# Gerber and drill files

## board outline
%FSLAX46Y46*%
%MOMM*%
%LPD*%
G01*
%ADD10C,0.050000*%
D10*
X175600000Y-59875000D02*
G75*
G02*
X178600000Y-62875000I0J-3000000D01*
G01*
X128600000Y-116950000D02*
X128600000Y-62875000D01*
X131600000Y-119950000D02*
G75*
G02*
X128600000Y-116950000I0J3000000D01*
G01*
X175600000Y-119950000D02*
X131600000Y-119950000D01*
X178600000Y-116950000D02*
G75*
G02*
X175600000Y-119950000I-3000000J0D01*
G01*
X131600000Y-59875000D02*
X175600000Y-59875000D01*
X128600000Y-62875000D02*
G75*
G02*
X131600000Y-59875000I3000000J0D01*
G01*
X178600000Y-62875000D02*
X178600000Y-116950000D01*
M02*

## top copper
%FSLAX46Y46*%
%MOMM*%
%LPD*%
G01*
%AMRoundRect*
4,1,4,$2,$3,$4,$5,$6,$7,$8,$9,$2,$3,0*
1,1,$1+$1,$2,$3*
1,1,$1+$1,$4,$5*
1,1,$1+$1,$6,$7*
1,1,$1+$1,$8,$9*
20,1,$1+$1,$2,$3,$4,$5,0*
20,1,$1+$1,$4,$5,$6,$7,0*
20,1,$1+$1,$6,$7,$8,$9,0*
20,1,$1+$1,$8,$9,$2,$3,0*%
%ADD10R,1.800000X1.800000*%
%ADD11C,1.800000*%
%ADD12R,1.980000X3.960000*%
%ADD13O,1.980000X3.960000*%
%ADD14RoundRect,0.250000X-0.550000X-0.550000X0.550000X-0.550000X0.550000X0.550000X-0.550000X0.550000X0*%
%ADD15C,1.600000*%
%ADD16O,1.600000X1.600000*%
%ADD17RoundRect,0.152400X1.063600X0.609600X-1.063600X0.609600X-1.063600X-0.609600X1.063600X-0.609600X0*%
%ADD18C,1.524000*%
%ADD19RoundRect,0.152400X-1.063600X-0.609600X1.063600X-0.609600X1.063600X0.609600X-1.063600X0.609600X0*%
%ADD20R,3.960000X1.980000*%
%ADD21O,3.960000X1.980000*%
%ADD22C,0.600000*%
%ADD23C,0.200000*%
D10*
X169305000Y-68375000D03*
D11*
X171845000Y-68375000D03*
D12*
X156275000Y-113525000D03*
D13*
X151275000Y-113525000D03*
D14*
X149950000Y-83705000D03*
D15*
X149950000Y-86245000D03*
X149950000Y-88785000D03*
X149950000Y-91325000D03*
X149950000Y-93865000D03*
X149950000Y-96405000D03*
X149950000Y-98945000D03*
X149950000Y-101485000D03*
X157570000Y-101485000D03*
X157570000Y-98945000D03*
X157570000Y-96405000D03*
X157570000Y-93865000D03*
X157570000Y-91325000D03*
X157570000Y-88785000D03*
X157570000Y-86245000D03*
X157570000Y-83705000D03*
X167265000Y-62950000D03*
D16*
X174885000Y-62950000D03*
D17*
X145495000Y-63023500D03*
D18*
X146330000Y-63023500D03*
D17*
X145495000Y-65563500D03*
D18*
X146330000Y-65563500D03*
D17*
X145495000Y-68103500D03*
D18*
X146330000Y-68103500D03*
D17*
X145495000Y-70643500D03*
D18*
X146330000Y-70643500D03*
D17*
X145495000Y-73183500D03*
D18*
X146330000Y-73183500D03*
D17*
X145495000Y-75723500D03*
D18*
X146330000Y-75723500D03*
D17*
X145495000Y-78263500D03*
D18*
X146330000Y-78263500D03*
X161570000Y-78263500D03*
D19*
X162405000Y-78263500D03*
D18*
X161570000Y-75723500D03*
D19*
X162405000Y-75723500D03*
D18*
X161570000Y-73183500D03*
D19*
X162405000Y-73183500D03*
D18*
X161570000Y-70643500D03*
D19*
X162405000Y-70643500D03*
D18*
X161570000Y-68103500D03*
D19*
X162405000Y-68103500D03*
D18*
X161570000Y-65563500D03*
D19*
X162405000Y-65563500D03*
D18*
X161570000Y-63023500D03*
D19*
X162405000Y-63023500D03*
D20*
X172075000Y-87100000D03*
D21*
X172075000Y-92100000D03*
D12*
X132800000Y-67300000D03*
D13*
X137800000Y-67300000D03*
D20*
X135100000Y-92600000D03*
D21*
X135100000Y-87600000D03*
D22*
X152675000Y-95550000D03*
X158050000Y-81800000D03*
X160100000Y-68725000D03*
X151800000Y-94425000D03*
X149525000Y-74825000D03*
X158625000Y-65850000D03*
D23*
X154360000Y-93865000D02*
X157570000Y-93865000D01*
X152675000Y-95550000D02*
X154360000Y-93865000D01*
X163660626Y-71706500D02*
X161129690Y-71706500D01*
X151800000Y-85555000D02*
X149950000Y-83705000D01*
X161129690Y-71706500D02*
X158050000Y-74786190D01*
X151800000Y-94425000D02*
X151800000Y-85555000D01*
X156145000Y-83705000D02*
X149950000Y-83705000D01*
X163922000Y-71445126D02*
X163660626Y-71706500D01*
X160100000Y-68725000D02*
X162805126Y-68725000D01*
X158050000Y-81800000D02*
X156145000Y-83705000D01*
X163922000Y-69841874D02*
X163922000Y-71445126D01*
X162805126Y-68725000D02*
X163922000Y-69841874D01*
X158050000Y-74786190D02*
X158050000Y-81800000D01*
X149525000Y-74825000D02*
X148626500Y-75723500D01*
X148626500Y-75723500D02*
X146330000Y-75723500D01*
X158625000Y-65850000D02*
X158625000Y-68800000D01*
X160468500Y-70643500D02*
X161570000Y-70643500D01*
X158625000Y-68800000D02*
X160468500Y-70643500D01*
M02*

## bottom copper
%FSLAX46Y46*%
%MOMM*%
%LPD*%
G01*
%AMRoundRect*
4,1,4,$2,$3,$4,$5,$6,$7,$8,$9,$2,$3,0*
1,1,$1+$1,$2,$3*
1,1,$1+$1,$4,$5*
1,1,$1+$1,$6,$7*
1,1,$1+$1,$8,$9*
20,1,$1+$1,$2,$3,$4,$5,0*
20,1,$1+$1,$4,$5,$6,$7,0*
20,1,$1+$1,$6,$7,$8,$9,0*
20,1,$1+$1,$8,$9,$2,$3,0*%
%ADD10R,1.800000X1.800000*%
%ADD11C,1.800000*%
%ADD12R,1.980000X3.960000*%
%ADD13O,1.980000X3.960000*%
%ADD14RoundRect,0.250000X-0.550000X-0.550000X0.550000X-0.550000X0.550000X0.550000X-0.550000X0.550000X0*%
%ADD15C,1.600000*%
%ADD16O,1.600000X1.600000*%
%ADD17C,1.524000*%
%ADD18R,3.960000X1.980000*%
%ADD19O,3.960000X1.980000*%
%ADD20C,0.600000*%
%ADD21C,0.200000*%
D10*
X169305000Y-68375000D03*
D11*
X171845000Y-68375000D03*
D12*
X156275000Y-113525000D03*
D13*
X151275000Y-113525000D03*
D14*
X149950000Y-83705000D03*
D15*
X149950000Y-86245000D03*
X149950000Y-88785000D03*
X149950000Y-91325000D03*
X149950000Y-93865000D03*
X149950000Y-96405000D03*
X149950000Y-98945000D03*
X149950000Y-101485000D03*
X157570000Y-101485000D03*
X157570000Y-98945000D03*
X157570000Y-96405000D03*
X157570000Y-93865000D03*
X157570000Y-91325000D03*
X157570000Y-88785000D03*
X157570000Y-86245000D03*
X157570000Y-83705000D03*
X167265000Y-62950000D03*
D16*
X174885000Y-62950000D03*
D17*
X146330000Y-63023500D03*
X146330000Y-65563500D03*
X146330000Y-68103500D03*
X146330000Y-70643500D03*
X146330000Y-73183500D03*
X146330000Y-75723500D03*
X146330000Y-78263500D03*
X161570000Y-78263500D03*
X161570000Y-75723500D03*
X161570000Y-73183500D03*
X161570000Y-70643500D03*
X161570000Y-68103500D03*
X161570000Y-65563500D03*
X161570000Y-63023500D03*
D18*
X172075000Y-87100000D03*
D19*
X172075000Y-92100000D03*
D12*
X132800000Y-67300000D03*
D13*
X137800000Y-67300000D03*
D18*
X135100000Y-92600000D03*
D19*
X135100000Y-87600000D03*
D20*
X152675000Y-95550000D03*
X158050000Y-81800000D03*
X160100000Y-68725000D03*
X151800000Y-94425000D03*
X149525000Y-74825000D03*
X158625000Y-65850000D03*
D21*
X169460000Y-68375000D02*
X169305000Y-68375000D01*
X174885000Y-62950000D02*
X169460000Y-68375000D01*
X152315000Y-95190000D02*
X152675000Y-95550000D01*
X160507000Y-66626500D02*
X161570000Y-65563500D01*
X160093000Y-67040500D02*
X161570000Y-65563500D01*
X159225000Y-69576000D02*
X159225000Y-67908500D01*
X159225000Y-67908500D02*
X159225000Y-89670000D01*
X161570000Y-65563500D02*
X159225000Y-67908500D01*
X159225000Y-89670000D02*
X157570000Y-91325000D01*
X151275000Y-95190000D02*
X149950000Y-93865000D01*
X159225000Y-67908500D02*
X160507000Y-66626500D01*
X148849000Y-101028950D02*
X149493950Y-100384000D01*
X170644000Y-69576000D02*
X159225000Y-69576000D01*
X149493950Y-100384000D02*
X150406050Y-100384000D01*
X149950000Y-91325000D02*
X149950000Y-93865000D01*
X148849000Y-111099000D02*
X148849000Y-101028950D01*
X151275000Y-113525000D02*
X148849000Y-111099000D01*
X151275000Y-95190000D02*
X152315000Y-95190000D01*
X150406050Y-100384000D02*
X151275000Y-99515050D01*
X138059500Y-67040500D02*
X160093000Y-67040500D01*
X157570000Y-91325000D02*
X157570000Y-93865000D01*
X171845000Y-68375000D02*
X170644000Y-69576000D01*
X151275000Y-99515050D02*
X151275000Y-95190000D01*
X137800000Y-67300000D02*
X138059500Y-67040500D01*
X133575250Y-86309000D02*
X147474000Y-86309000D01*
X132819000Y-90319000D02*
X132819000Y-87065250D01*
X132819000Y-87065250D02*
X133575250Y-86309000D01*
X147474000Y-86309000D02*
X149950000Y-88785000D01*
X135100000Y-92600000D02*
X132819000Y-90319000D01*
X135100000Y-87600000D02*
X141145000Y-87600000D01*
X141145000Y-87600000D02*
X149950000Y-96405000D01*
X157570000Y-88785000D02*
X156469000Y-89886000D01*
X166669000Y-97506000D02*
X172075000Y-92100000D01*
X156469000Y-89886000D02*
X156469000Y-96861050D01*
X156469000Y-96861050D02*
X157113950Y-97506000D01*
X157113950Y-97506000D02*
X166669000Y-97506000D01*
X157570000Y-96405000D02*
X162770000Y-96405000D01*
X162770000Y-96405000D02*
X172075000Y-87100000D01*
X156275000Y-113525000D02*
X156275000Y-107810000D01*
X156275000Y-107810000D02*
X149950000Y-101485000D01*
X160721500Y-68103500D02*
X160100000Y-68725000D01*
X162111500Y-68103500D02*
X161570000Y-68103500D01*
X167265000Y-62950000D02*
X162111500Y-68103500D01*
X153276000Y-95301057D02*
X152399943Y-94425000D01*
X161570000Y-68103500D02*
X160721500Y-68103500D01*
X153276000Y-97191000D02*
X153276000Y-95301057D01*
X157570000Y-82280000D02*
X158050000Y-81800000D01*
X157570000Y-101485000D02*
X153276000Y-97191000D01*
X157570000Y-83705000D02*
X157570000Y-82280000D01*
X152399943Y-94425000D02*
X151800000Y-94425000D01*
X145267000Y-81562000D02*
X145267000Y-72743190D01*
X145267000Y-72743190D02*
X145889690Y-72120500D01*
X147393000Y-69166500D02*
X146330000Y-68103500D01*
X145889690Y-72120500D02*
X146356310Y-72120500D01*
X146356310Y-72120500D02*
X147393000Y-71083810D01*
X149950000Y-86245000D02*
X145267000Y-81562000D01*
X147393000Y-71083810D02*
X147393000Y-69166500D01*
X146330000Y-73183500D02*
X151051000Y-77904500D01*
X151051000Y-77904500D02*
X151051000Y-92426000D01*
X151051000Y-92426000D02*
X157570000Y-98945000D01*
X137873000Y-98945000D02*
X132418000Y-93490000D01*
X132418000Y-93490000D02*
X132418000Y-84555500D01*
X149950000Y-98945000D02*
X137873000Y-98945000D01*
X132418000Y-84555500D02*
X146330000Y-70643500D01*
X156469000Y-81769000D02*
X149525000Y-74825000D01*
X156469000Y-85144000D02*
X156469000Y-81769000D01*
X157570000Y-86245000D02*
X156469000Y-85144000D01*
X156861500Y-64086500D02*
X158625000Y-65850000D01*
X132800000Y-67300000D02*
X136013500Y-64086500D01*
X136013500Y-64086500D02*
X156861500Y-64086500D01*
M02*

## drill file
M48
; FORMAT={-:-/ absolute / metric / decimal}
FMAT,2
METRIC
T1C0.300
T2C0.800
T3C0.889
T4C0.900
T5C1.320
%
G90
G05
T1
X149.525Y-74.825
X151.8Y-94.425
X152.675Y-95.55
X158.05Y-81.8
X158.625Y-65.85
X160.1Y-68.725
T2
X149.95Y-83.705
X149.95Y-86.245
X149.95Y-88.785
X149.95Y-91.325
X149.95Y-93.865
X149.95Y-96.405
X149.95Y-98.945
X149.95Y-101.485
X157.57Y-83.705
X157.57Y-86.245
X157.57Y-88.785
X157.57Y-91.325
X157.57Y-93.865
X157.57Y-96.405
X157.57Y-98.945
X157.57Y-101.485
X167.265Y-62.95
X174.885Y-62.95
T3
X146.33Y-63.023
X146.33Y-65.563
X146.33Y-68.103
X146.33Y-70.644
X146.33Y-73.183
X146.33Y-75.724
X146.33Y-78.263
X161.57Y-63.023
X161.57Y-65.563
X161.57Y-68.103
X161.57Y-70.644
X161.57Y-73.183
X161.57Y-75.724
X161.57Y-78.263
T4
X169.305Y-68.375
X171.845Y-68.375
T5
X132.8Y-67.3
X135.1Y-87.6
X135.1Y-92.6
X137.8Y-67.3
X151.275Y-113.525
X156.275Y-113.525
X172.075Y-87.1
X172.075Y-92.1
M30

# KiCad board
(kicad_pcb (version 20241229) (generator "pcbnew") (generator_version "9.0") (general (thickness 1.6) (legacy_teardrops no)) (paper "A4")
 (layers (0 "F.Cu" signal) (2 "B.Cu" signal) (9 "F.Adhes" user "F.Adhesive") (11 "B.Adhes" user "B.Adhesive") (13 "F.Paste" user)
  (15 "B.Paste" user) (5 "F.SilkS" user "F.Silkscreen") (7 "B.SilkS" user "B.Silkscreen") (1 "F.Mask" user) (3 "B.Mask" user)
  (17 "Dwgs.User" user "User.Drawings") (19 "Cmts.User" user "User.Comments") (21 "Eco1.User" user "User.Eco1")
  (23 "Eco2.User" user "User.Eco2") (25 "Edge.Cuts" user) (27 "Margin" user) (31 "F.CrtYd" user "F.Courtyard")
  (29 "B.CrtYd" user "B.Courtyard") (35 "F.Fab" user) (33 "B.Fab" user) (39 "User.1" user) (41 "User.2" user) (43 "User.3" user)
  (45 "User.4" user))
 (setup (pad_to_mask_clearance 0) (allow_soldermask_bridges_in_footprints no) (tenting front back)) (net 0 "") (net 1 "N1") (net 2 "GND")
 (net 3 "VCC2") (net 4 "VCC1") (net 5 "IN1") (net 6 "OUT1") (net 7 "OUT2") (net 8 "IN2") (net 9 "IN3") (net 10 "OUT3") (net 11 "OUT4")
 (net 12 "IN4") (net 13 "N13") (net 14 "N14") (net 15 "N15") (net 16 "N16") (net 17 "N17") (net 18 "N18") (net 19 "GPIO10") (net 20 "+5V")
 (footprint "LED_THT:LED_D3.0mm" (layer "F.Cu") (at 169.305 68.375)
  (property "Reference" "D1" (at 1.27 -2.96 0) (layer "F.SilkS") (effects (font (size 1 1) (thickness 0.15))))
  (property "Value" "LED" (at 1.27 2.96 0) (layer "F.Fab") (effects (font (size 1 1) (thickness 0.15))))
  (pad "1" thru_hole rect (at 0 0) (size 1.8 1.8) (drill 0.9) (layers "*.Cu" "*.Mask") (remove_unused_layers no) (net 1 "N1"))
  (pad "2" thru_hole circle (at 2.54 0) (size 1.8 1.8) (drill 0.9) (layers "*.Cu" "*.Mask") (remove_unused_layers no) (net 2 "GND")))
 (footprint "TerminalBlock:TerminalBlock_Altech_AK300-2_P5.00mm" (layer "F.Cu") (at 156.275 113.525 180)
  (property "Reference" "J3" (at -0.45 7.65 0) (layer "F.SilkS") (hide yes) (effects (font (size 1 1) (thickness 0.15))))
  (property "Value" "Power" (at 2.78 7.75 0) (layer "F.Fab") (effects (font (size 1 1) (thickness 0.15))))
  (pad "1" thru_hole rect (at 0 0 180) (size 1.98 3.96) (drill 1.32) (layers "*.Cu" "*.Mask") (remove_unused_layers no) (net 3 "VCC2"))
  (pad "2" thru_hole oval (at 5 0 180) (size 1.98 3.96) (drill 1.32) (layers "*.Cu" "*.Mask") (remove_unused_layers no) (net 2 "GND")))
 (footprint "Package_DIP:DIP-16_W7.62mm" (layer "F.Cu") (at 149.95 83.705)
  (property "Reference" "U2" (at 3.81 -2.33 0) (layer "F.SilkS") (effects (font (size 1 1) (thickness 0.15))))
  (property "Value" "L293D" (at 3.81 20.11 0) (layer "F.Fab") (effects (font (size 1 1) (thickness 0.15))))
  (pad "1" thru_hole roundrect (at 0 0) (size 1.6 1.6) (drill 0.8) (layers "*.Cu" "*.Mask") (remove_unused_layers no)
   (roundrect_rratio 0.15625) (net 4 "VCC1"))
  (pad "2" thru_hole circle (at 0 2.54) (size 1.6 1.6) (drill 0.8) (layers "*.Cu" "*.Mask") (remove_unused_layers no) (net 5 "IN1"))
  (pad "3" thru_hole circle (at 0 5.08) (size 1.6 1.6) (drill 0.8) (layers "*.Cu" "*.Mask") (remove_unused_layers no) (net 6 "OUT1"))
  (pad "4" thru_hole circle (at 0 7.62) (size 1.6 1.6) (drill 0.8) (layers "*.Cu" "*.Mask") (remove_unused_layers no) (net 2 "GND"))
  (pad "5" thru_hole circle (at 0 10.16) (size 1.6 1.6) (drill 0.8) (layers "*.Cu" "*.Mask") (remove_unused_layers no) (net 2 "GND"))
  (pad "6" thru_hole circle (at 0 12.7) (size 1.6 1.6) (drill 0.8) (layers "*.Cu" "*.Mask") (remove_unused_layers no) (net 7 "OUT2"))
  (pad "7" thru_hole circle (at 0 15.24) (size 1.6 1.6) (drill 0.8) (layers "*.Cu" "*.Mask") (remove_unused_layers no) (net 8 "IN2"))
  (pad "8" thru_hole circle (at 0 17.78) (size 1.6 1.6) (drill 0.8) (layers "*.Cu" "*.Mask") (remove_unused_layers no) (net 3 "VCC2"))
  (pad "9" thru_hole circle (at 7.62 17.78) (size 1.6 1.6) (drill 0.8) (layers "*.Cu" "*.Mask") (remove_unused_layers no) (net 4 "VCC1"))
  (pad "10" thru_hole circle (at 7.62 15.24) (size 1.6 1.6) (drill 0.8) (layers "*.Cu" "*.Mask") (remove_unused_layers no) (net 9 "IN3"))
  (pad "11" thru_hole circle (at 7.62 12.7) (size 1.6 1.6) (drill 0.8) (layers "*.Cu" "*.Mask") (remove_unused_layers no) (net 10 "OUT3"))
  (pad "12" thru_hole circle (at 7.62 10.16) (size 1.6 1.6) (drill 0.8) (layers "*.Cu" "*.Mask") (remove_unused_layers no) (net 2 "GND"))
  (pad "13" thru_hole circle (at 7.62 7.62) (size 1.6 1.6) (drill 0.8) (layers "*.Cu" "*.Mask") (remove_unused_layers no) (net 2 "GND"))
  (pad "14" thru_hole circle (at 7.62 5.08) (size 1.6 1.6) (drill 0.8) (layers "*.Cu" "*.Mask") (remove_unused_layers no) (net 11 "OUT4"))
  (pad "15" thru_hole circle (at 7.62 2.54) (size 1.6 1.6) (drill 0.8) (layers "*.Cu" "*.Mask") (remove_unused_layers no) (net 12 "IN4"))
  (pad "16" thru_hole circle (at 7.62 0) (size 1.6 1.6) (drill 0.8) (layers "*.Cu" "*.Mask") (remove_unused_layers no) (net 4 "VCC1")))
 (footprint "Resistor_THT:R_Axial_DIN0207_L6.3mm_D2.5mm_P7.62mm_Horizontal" (layer "F.Cu") (at 167.265 62.95)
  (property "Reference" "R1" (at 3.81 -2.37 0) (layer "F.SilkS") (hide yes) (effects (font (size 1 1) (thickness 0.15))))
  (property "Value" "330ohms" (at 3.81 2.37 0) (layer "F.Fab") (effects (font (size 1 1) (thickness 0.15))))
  (pad "1" thru_hole circle (at 0 0) (size 1.6 1.6) (drill 0.8) (layers "*.Cu" "*.Mask") (remove_unused_layers no) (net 4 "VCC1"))
  (pad "2" thru_hole oval (at 7.62 0) (size 1.6 1.6) (drill 0.8) (layers "*.Cu" "*.Mask") (remove_unused_layers no) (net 1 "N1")))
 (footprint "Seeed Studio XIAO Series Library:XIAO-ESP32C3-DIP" (layer "F.Cu") (at 154.07 70.6435)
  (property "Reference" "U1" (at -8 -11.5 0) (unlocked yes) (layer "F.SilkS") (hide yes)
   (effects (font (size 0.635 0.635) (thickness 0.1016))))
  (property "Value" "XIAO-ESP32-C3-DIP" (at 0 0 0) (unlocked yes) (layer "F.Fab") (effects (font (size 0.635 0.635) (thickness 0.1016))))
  (pad "1" smd roundrect (at -8.575 -7.62 180) (size 2.432 1.524) (layers "F.Cu" "F.Mask") (roundrect_rratio 0.1) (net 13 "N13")
   (thermal_bridge_angle 45))
  (pad "1" thru_hole circle (at -7.74 -7.62 180) (size 1.524 1.524) (drill 0.889) (layers "*.Cu" "*.Mask") (remove_unused_layers no)
   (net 13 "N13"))
  (pad "2" smd roundrect (at -8.575 -5.08 180) (size 2.432 1.524) (layers "F.Cu" "F.Mask") (roundrect_rratio 0.1) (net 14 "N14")
   (thermal_bridge_angle 45))
  (pad "2" thru_hole circle (at -7.74 -5.08 180) (size 1.524 1.524) (drill 0.889) (layers "*.Cu" "*.Mask") (remove_unused_layers no)
   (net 14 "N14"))
  (pad "3" smd roundrect (at -8.575 -2.54 180) (size 2.432 1.524) (layers "F.Cu" "F.Mask") (roundrect_rratio 0.1) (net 5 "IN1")
   (thermal_bridge_angle 45))
  (pad "3" thru_hole circle (at -7.74 -2.54 180) (size 1.524 1.524) (drill 0.889) (layers "*.Cu" "*.Mask") (remove_unused_layers no)
   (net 5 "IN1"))
  (pad "4" smd roundrect (at -8.575 0 180) (size 2.432 1.524) (layers "F.Cu" "F.Mask") (roundrect_rratio 0.1) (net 8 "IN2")
   (thermal_bridge_angle 45))
  (pad "4" thru_hole circle (at -7.74 0 180) (size 1.524 1.524) (drill 0.889) (layers "*.Cu" "*.Mask") (remove_unused_layers no)
   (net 8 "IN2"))
  (pad "5" smd roundrect (at -8.575 2.54 180) (size 2.432 1.524) (layers "F.Cu" "F.Mask") (roundrect_rratio 0.1) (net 9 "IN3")
   (thermal_bridge_angle 45))
  (pad "5" thru_hole circle (at -7.74 2.54 180) (size 1.524 1.524) (drill 0.889) (layers "*.Cu" "*.Mask") (remove_unused_layers no)
   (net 9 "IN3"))
  (pad "6" smd roundrect (at -8.575 5.08 180) (size 2.432 1.524) (layers "F.Cu" "F.Mask") (roundrect_rratio 0.1) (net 12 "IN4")
   (thermal_bridge_angle 45))
  (pad "6" thru_hole circle (at -7.74 5.08 180) (size 1.524 1.524) (drill 0.889) (layers "*.Cu" "*.Mask") (remove_unused_layers no)
   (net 12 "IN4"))
  (pad "7" smd roundrect (at -8.575 7.62 180) (size 2.432 1.524) (layers "F.Cu" "F.Mask") (roundrect_rratio 0.1) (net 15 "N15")
   (thermal_bridge_angle 45))
  (pad "7" thru_hole circle (at -7.74 7.62 180) (size 1.524 1.524) (drill 0.889) (layers "*.Cu" "*.Mask") (remove_unused_layers no)
   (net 15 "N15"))
  (pad "8" thru_hole circle (at 7.5 7.62) (size 1.524 1.524) (drill 0.889) (layers "*.Cu" "*.Mask") (remove_unused_layers no) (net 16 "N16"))
  (pad "8" smd roundrect (at 8.335 7.62) (size 2.432 1.524) (layers "F.Cu" "F.Mask") (roundrect_rratio 0.1) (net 16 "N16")
   (thermal_bridge_angle 45))
  (pad "9" thru_hole circle (at 7.5 5.08) (size 1.524 1.524) (drill 0.889) (layers "*.Cu" "*.Mask") (remove_unused_layers no) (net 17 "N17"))
  (pad "9" smd roundrect (at 8.335 5.08) (size 2.432 1.524) (layers "F.Cu" "F.Mask") (roundrect_rratio 0.1) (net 17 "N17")
   (thermal_bridge_angle 45))
  (pad "10" thru_hole circle (at 7.5 2.54) (size 1.524 1.524) (drill 0.889) (layers "*.Cu" "*.Mask") (remove_unused_layers no)
   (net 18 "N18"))
  (pad "10" smd roundrect (at 8.335 2.54) (size 2.432 1.524) (layers "F.Cu" "F.Mask") (roundrect_rratio 0.1) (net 18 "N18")
   (thermal_bridge_angle 45))
  (pad "11" thru_hole circle (at 7.5 0) (size 1.524 1.524) (drill 0.889) (layers "*.Cu" "*.Mask") (remove_unused_layers no)
   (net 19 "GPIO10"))
  (pad "11" smd roundrect (at 8.335 0) (size 2.432 1.524) (layers "F.Cu" "F.Mask") (roundrect_rratio 0.1) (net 19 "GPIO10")
   (thermal_bridge_angle 45))
  (pad "12" thru_hole circle (at 7.5 -2.54) (size 1.524 1.524) (drill 0.889) (layers "*.Cu" "*.Mask") (remove_unused_layers no)
   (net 4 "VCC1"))
  (pad "12" smd roundrect (at 8.335 -2.54) (size 2.432 1.524) (layers "F.Cu" "F.Mask") (roundrect_rratio 0.1) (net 4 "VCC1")
   (thermal_bridge_angle 45))
  (pad "13" thru_hole circle (at 7.5 -5.08) (size 1.524 1.524) (drill 0.889) (layers "*.Cu" "*.Mask") (remove_unused_layers no)
   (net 2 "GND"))
  (pad "13" smd roundrect (at 8.335 -5.08) (size 2.432 1.524) (layers "F.Cu" "F.Mask") (roundrect_rratio 0.1) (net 2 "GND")
   (thermal_bridge_angle 45))
  (pad "14" thru_hole circle (at 7.5 -7.62) (size 1.524 1.524) (drill 0.889) (layers "*.Cu" "*.Mask") (remove_unused_layers no)
   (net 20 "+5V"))
  (pad "14" smd roundrect (at 8.335 -7.62) (size 2.432 1.524) (layers "F.Cu" "F.Mask") (roundrect_rratio 0.1) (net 20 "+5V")
   (thermal_bridge_angle 45)))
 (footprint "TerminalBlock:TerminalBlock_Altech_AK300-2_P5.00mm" (layer "F.Cu") (at 172.075 87.1 -90)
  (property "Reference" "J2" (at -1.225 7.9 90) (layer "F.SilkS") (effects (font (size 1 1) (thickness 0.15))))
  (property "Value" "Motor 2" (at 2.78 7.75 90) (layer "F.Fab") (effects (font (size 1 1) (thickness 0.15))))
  (pad "1" thru_hole rect (at 0 0 270) (size 1.98 3.96) (drill 1.32) (layers "*.Cu" "*.Mask") (remove_unused_layers no) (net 10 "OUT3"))
  (pad "2" thru_hole oval (at 5 0 270) (size 1.98 3.96) (drill 1.32) (layers "*.Cu" "*.Mask") (remove_unused_layers no) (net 11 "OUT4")))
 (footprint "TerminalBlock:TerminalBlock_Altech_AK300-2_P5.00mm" (layer "F.Cu") (at 132.8 67.3)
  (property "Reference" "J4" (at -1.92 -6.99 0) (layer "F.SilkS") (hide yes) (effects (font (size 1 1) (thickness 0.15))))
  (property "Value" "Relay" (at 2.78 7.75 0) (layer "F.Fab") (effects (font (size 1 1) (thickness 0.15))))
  (pad "1" thru_hole rect (at 0 0) (size 1.98 3.96) (drill 1.32) (layers "*.Cu" "*.Mask") (remove_unused_layers no) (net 19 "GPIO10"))
  (pad "2" thru_hole oval (at 5 0) (size 1.98 3.96) (drill 1.32) (layers "*.Cu" "*.Mask") (remove_unused_layers no) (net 2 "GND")))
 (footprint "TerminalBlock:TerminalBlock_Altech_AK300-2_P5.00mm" (layer "F.Cu") (at 135.1 92.6 90)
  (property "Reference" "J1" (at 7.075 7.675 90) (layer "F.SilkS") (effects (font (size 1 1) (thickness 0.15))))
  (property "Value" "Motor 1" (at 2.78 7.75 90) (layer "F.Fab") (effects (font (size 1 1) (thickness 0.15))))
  (pad "1" thru_hole rect (at 0 0 90) (size 1.98 3.96) (drill 1.32) (layers "*.Cu" "*.Mask") (remove_unused_layers no) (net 6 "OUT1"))
  (pad "2" thru_hole oval (at 5 0 90) (size 1.98 3.96) (drill 1.32) (layers "*.Cu" "*.Mask") (remove_unused_layers no) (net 7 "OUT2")))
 (gr_arc (start 175.6 59.875) (mid 177.72132 60.75368) (end 178.6 62.875) (stroke (width 0.05) (type default)) (layer "Edge.Cuts"))
 (gr_line (start 128.6 116.95) (end 128.6 62.875) (stroke (width 0.05) (type default)) (layer "Edge.Cuts"))
 (gr_arc (start 131.6 119.95) (mid 129.47868 119.07132) (end 128.6 116.95) (stroke (width 0.05) (type default)) (layer "Edge.Cuts"))
 (gr_line (start 175.6 119.95) (end 131.6 119.95) (stroke (width 0.05) (type default)) (layer "Edge.Cuts"))
 (gr_arc (start 178.6 116.95) (mid 177.72132 119.07132) (end 175.6 119.95) (stroke (width 0.05) (type default)) (layer "Edge.Cuts"))
 (gr_line (start 131.6 59.875) (end 175.6 59.875) (stroke (width 0.05) (type default)) (layer "Edge.Cuts"))
 (gr_arc (start 128.6 62.875) (mid 129.47868 60.75368) (end 131.6 59.875) (stroke (width 0.05) (type default)) (layer "Edge.Cuts"))
 (gr_line (start 178.6 62.875) (end 178.6 116.95) (stroke (width 0.05) (type default)) (layer "Edge.Cuts"))
 (segment (start 169.46 68.375) (end 169.305 68.375) (width 0.2) (layer "B.Cu") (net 1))
 (segment (start 174.885 62.95) (end 169.46 68.375) (width 0.2) (layer "B.Cu") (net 1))
 (segment (start 154.36 93.865) (end 157.57 93.865) (width 0.2) (layer "F.Cu") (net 2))
 (segment (start 152.675 95.55) (end 154.36 93.865) (width 0.2) (layer "F.Cu") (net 2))
 (via (at 152.675 95.55) (size 0.6) (drill 0.3) (layers "F.Cu" "B.Cu") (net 2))
 (segment (start 152.315 95.19) (end 152.675 95.55) (width 0.2) (layer "B.Cu") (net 2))
 (segment (start 160.507 66.6265) (end 161.57 65.5635) (width 0.2) (layer "B.Cu") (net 2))
 (segment (start 160.093 67.0405) (end 161.57 65.5635) (width 0.2) (layer "B.Cu") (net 2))
 (segment (start 159.225 69.576) (end 159.225 67.9085) (width 0.2) (layer "B.Cu") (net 2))
 (segment (start 159.225 67.9085) (end 159.225 89.67) (width 0.2) (layer "B.Cu") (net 2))
 (segment (start 161.57 65.5635) (end 159.225 67.9085) (width 0.2) (layer "B.Cu") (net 2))
 (segment (start 159.225 89.67) (end 157.57 91.325) (width 0.2) (layer "B.Cu") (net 2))
 (segment (start 151.275 95.19) (end 149.95 93.865) (width 0.2) (layer "B.Cu") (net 2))
 (segment (start 159.225 67.9085) (end 160.507 66.6265) (width 0.2) (layer "B.Cu") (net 2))
 (segment (start 148.849 101.02895) (end 149.49395 100.384) (width 0.2) (layer "B.Cu") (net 2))
 (segment (start 170.644 69.576) (end 159.225 69.576) (width 0.2) (layer "B.Cu") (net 2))
 (segment (start 149.49395 100.384) (end 150.40605 100.384) (width 0.2) (layer "B.Cu") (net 2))
 (segment (start 149.95 91.325) (end 149.95 93.865) (width 0.2) (layer "B.Cu") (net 2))
 (segment (start 148.849 111.099) (end 148.849 101.02895) (width 0.2) (layer "B.Cu") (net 2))
 (segment (start 151.275 113.525) (end 148.849 111.099) (width 0.2) (layer "B.Cu") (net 2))
 (segment (start 151.275 95.19) (end 152.315 95.19) (width 0.2) (layer "B.Cu") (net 2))
 (segment (start 150.40605 100.384) (end 151.275 99.51505) (width 0.2) (layer "B.Cu") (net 2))
 (segment (start 138.0595 67.0405) (end 160.093 67.0405) (width 0.2) (layer "B.Cu") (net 2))
 (segment (start 157.57 91.325) (end 157.57 93.865) (width 0.2) (layer "B.Cu") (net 2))
 (segment (start 171.845 68.375) (end 170.644 69.576) (width 0.2) (layer "B.Cu") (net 2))
 (segment (start 151.275 99.51505) (end 151.275 95.19) (width 0.2) (layer "B.Cu") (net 2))
 (segment (start 137.8 67.3) (end 138.0595 67.0405) (width 0.2) (layer "B.Cu") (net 2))
 (segment (start 133.57525 86.309) (end 147.474 86.309) (width 0.2) (layer "B.Cu") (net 6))
 (segment (start 132.819 90.319) (end 132.819 87.06525) (width 0.2) (layer "B.Cu") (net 6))
 (segment (start 132.819 87.06525) (end 133.57525 86.309) (width 0.2) (layer "B.Cu") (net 6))
 (segment (start 147.474 86.309) (end 149.95 88.785) (width 0.2) (layer "B.Cu") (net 6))
 (segment (start 135.1 92.6) (end 132.819 90.319) (width 0.2) (layer "B.Cu") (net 6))
 (segment (start 135.1 87.6) (end 141.145 87.6) (width 0.2) (layer "B.Cu") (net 7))
 (segment (start 141.145 87.6) (end 149.95 96.405) (width 0.2) (layer "B.Cu") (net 7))
 (segment (start 157.57 88.785) (end 156.469 89.886) (width 0.2) (layer "B.Cu") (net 11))
 (segment (start 166.669 97.506) (end 172.075 92.1) (width 0.2) (layer "B.Cu") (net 11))
 (segment (start 156.469 89.886) (end 156.469 96.86105) (width 0.2) (layer "B.Cu") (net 11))
 (segment (start 156.469 96.86105) (end 157.11395 97.506) (width 0.2) (layer "B.Cu") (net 11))
 (segment (start 157.11395 97.506) (end 166.669 97.506) (width 0.2) (layer "B.Cu") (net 11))
 (segment (start 157.57 96.405) (end 162.77 96.405) (width 0.2) (layer "B.Cu") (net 10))
 (segment (start 162.77 96.405) (end 172.075 87.1) (width 0.2) (layer "B.Cu") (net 10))
 (segment (start 156.275 113.525) (end 156.275 107.81) (width 0.2) (layer "B.Cu") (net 3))
 (segment (start 156.275 107.81) (end 149.95 101.485) (width 0.2) (layer "B.Cu") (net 3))
 (segment (start 163.660626 71.7065) (end 161.12969 71.7065) (width 0.2) (layer "F.Cu") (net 4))
 (segment (start 151.8 85.555) (end 149.95 83.705) (width 0.2) (layer "F.Cu") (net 4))
 (segment (start 161.12969 71.7065) (end 158.05 74.78619) (width 0.2) (layer "F.Cu") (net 4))
 (segment (start 151.8 94.425) (end 151.8 85.555) (width 0.2) (layer "F.Cu") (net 4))
 (segment (start 156.145 83.705) (end 149.95 83.705) (width 0.2) (layer "F.Cu") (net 4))
 (segment (start 163.922 71.445126) (end 163.660626 71.7065) (width 0.2) (layer "F.Cu") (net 4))
 (segment (start 160.1 68.725) (end 162.805126 68.725) (width 0.2) (layer "F.Cu") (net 4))
 (segment (start 158.05 81.8) (end 156.145 83.705) (width 0.2) (layer "F.Cu") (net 4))
 (segment (start 163.922 69.841874) (end 163.922 71.445126) (width 0.2) (layer "F.Cu") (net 4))
 (segment (start 162.805126 68.725) (end 163.922 69.841874) (width 0.2) (layer "F.Cu") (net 4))
 (segment (start 158.05 74.78619) (end 158.05 81.8) (width 0.2) (layer "F.Cu") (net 4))
 (via (at 158.05 81.8) (size 0.6) (drill 0.3) (layers "F.Cu" "B.Cu") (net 4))
 (via (at 160.1 68.725) (size 0.6) (drill 0.3) (layers "F.Cu" "B.Cu") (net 4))
 (via (at 151.8 94.425) (size 0.6) (drill 0.3) (layers "F.Cu" "B.Cu") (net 4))
 (segment (start 160.7215 68.1035) (end 160.1 68.725) (width 0.2) (layer "B.Cu") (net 4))
 (segment (start 162.1115 68.1035) (end 161.57 68.1035) (width 0.2) (layer "B.Cu") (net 4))
 (segment (start 167.265 62.95) (end 162.1115 68.1035) (width 0.2) (layer "B.Cu") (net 4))
 (segment (start 153.276 95.301057) (end 152.399943 94.425) (width 0.2) (layer "B.Cu") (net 4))
 (segment (start 161.57 68.1035) (end 160.7215 68.1035) (width 0.2) (layer "B.Cu") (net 4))
 (segment (start 153.276 97.191) (end 153.276 95.301057) (width 0.2) (layer "B.Cu") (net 4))
 (segment (start 157.57 82.28) (end 158.05 81.8) (width 0.2) (layer "B.Cu") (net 4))
 (segment (start 157.57 101.485) (end 153.276 97.191) (width 0.2) (layer "B.Cu") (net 4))
 (segment (start 157.57 83.705) (end 157.57 82.28) (width 0.2) (layer "B.Cu") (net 4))
 (segment (start 152.399943 94.425) (end 151.8 94.425) (width 0.2) (layer "B.Cu") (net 4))
 (segment (start 145.267 81.562) (end 145.267 72.74319) (width 0.2) (layer "B.Cu") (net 5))
 (segment (start 145.267 72.74319) (end 145.88969 72.1205) (width 0.2) (layer "B.Cu") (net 5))
 (segment (start 147.393 69.1665) (end 146.33 68.1035) (width 0.2) (layer "B.Cu") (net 5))
 (segment (start 145.88969 72.1205) (end 146.35631 72.1205) (width 0.2) (layer "B.Cu") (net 5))
 (segment (start 146.35631 72.1205) (end 147.393 71.08381) (width 0.2) (layer "B.Cu") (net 5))
 (segment (start 149.95 86.245) (end 145.267 81.562) (width 0.2) (layer "B.Cu") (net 5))
 (segment (start 147.393 71.08381) (end 147.393 69.1665) (width 0.2) (layer "B.Cu") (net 5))
 (segment (start 146.33 73.1835) (end 151.051 77.9045) (width 0.2) (layer "B.Cu") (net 9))
 (segment (start 151.051 77.9045) (end 151.051 92.426) (width 0.2) (layer "B.Cu") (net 9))
 (segment (start 151.051 92.426) (end 157.57 98.945) (width 0.2) (layer "B.Cu") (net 9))
 (segment (start 137.873 98.945) (end 132.418 93.49) (width 0.2) (layer "B.Cu") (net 8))
 (segment (start 132.418 93.49) (end 132.418 84.5555) (width 0.2) (layer "B.Cu") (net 8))
 (segment (start 149.95 98.945) (end 137.873 98.945) (width 0.2) (layer "B.Cu") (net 8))
 (segment (start 132.418 84.5555) (end 146.33 70.6435) (width 0.2) (layer "B.Cu") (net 8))
 (segment (start 149.525 74.825) (end 148.6265 75.7235) (width 0.2) (layer "F.Cu") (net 12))
 (segment (start 148.6265 75.7235) (end 146.33 75.7235) (width 0.2) (layer "F.Cu") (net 12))
 (via (at 149.525 74.825) (size 0.6) (drill 0.3) (layers "F.Cu" "B.Cu") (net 12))
 (segment (start 156.469 81.769) (end 149.525 74.825) (width 0.2) (layer "B.Cu") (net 12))
 (segment (start 156.469 85.144) (end 156.469 81.769) (width 0.2) (layer "B.Cu") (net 12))
 (segment (start 157.57 86.245) (end 156.469 85.144) (width 0.2) (layer "B.Cu") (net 12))
 (segment (start 158.625 65.85) (end 158.625 68.8) (width 0.2) (layer "F.Cu") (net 19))
 (segment (start 160.4685 70.6435) (end 161.57 70.6435) (width 0.2) (layer "F.Cu") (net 19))
 (segment (start 158.625 68.8) (end 160.4685 70.6435) (width 0.2) (layer "F.Cu") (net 19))
 (via (at 158.625 65.85) (size 0.6) (drill 0.3) (layers "F.Cu" "B.Cu") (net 19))
 (segment (start 156.8615 64.0865) (end 158.625 65.85) (width 0.2) (layer "B.Cu") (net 19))
 (segment (start 132.8 67.3) (end 136.0135 64.0865) (width 0.2) (layer "B.Cu") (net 19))
 (segment (start 136.0135 64.0865) (end 156.8615 64.0865) (width 0.2) (layer "B.Cu") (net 19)))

